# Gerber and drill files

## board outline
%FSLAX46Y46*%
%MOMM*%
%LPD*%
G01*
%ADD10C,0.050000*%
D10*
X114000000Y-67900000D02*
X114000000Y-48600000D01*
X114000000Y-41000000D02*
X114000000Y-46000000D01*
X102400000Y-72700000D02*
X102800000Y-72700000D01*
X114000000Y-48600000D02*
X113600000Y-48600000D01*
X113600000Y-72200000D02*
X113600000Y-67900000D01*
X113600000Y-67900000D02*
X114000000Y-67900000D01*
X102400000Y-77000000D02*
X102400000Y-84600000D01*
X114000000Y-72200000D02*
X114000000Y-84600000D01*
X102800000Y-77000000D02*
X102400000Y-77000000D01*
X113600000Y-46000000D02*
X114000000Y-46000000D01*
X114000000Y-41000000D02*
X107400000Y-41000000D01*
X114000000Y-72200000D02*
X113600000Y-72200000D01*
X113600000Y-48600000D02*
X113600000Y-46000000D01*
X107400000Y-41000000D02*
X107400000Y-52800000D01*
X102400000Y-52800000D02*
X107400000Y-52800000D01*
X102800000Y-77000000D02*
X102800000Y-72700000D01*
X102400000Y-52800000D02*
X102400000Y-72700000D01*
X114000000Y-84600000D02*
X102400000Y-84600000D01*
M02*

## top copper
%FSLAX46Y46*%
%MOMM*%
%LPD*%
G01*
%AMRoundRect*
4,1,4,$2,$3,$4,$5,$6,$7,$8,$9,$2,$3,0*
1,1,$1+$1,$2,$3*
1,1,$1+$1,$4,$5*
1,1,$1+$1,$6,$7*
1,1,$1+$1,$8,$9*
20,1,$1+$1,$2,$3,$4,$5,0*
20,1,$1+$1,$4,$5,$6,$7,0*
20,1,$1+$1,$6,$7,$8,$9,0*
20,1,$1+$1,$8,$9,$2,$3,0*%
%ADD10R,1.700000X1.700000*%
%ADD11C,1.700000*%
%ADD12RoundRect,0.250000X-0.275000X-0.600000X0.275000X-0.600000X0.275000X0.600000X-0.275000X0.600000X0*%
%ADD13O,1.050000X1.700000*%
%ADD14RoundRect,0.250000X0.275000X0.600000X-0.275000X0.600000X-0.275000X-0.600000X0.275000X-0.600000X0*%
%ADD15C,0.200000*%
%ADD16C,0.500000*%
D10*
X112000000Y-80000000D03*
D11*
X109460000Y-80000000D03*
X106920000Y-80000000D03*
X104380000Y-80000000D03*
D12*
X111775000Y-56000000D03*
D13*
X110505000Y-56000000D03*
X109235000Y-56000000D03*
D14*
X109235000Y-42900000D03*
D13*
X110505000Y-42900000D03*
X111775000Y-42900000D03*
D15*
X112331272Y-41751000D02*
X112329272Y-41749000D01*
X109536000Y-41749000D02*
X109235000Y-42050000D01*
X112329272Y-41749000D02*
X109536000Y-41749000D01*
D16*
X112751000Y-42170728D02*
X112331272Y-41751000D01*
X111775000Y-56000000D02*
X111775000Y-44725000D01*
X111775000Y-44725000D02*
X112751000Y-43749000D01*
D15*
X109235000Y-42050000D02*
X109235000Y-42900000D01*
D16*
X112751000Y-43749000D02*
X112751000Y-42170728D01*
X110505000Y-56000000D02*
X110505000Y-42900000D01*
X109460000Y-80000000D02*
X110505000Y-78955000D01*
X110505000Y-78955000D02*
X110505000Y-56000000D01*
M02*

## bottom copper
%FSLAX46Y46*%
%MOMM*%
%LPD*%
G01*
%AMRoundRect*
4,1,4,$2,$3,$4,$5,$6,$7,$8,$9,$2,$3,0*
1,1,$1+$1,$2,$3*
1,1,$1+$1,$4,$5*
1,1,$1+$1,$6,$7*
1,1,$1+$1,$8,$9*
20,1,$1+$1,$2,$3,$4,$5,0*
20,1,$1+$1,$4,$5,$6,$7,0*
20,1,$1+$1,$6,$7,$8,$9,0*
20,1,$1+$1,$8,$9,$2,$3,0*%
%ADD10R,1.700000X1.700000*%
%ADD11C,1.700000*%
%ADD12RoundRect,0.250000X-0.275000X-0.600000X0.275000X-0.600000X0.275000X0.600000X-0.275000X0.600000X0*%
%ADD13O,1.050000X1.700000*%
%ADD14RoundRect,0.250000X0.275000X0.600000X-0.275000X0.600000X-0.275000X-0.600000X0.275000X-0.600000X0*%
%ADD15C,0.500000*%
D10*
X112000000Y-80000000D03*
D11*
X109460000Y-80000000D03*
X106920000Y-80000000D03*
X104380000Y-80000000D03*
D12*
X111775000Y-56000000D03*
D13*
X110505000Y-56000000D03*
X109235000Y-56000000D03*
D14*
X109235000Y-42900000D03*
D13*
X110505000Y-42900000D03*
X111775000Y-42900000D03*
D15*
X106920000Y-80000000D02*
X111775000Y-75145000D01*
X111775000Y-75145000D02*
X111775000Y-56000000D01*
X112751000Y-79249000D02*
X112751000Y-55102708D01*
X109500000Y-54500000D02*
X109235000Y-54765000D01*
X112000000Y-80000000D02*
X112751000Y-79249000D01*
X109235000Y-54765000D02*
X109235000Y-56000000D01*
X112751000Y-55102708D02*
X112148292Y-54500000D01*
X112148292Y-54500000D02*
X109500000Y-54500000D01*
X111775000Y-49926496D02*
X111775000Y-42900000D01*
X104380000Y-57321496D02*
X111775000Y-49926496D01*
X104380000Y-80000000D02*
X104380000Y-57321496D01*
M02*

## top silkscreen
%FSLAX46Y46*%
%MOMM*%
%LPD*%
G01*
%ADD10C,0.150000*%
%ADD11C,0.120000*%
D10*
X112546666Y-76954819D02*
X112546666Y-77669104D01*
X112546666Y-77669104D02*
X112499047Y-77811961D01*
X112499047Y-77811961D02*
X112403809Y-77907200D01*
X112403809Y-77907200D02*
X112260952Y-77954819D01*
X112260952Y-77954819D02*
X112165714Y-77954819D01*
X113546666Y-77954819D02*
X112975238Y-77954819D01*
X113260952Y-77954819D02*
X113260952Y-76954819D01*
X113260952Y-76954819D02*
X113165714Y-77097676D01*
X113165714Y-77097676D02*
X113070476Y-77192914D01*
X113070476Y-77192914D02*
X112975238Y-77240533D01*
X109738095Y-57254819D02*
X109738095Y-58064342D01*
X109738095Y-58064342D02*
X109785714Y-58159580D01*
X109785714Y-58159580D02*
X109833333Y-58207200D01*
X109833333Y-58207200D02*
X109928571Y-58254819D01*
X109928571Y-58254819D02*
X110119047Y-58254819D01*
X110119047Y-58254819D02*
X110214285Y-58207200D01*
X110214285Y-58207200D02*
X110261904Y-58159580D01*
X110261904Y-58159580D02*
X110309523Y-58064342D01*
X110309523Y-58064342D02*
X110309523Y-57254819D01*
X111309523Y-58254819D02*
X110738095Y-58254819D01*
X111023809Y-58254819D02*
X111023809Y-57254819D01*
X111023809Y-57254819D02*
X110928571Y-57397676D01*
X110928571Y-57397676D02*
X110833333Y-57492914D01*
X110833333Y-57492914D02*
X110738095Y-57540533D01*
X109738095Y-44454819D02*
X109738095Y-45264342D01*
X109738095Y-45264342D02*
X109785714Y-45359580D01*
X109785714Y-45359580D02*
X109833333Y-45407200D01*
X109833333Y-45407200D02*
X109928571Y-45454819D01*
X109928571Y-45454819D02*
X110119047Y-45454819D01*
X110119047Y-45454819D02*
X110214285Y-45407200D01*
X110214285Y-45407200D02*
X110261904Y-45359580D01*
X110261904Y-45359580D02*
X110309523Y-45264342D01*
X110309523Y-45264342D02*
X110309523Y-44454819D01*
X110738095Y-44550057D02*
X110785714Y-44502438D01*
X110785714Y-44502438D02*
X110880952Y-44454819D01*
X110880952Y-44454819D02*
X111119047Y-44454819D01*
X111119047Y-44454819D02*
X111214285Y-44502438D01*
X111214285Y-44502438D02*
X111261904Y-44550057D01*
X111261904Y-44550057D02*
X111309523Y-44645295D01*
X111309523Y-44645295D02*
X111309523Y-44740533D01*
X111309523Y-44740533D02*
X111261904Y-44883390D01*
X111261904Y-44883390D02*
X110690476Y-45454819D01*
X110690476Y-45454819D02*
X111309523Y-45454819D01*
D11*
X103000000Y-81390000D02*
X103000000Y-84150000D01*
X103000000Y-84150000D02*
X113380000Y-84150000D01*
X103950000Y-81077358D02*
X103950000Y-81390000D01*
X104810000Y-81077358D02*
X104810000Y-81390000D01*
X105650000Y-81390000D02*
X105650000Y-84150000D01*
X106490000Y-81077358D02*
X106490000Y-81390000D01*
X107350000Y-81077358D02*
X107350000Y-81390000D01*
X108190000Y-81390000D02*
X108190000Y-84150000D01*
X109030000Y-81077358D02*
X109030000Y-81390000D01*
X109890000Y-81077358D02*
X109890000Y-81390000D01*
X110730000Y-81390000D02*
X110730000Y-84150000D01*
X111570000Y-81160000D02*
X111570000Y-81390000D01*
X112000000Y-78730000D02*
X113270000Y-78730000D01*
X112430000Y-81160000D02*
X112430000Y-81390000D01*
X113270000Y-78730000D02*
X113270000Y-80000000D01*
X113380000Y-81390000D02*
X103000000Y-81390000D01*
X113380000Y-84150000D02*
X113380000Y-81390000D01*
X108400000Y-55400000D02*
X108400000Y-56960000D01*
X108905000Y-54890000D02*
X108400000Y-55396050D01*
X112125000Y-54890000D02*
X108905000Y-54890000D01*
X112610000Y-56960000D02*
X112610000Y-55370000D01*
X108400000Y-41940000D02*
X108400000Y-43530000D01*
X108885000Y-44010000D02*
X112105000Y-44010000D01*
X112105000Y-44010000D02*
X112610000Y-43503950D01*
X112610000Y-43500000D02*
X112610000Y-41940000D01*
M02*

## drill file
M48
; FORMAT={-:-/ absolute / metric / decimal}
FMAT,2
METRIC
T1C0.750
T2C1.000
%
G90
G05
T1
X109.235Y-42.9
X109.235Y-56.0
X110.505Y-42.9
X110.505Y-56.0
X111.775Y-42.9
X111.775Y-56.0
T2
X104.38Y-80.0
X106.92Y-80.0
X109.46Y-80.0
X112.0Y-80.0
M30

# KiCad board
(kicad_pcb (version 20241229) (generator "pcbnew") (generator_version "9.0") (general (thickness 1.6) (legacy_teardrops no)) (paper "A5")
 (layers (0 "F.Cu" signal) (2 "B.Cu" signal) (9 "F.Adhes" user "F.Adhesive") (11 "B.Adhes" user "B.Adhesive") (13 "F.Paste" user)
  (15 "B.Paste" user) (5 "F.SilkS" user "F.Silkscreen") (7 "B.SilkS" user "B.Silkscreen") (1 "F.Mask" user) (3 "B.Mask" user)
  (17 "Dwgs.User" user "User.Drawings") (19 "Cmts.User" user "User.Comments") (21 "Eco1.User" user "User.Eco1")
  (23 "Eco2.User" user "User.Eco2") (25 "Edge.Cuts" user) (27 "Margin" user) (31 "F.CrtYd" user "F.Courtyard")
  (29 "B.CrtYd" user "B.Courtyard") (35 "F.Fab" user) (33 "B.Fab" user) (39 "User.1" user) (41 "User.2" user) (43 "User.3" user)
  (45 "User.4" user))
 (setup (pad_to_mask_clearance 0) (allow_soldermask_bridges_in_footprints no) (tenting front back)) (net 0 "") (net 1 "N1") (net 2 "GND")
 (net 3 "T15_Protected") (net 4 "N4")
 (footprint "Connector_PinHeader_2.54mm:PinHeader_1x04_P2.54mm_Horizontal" (layer "F.Cu") (at 112 80 -90)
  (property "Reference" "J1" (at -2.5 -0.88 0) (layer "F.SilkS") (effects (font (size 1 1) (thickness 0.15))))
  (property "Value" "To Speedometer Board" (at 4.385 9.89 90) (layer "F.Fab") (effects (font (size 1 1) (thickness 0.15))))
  (fp_line (start 1.39 9) (end 4.15 9) (stroke (width 0.12) (type solid)) (layer "F.SilkS"))
  (fp_line (start 4.15 9) (end 4.15 -1.38) (stroke (width 0.12) (type solid)) (layer "F.SilkS"))
  (fp_line (start 1.077358 8.05) (end 1.39 8.05) (stroke (width 0.12) (type solid)) (layer "F.SilkS"))
  (fp_line (start 1.077358 7.19) (end 1.39 7.19) (stroke (width 0.12) (type solid)) (layer "F.SilkS"))
  (fp_line (start 1.39 6.35) (end 4.15 6.35) (stroke (width 0.12) (type solid)) (layer "F.SilkS"))
  (fp_line (start 1.077358 5.51) (end 1.39 5.51) (stroke (width 0.12) (type solid)) (layer "F.SilkS"))
  (fp_line (start 1.077358 4.65) (end 1.39 4.65) (stroke (width 0.12) (type solid)) (layer "F.SilkS"))
  (fp_line (start 1.39 3.81) (end 4.15 3.81) (stroke (width 0.12) (type solid)) (layer "F.SilkS"))
  (fp_line (start 1.077358 2.97) (end 1.39 2.97) (stroke (width 0.12) (type solid)) (layer "F.SilkS"))
  (fp_line (start 1.077358 2.11) (end 1.39 2.11) (stroke (width 0.12) (type solid)) (layer "F.SilkS"))
  (fp_line (start 1.39 1.27) (end 4.15 1.27) (stroke (width 0.12) (type solid)) (layer "F.SilkS"))
  (fp_line (start 1.16 0.43) (end 1.39 0.43) (stroke (width 0.12) (type solid)) (layer "F.SilkS"))
  (fp_line (start -1.27 0) (end -1.27 -1.27) (stroke (width 0.12) (type solid)) (layer "F.SilkS"))
  (fp_line (start 1.16 -0.43) (end 1.39 -0.43) (stroke (width 0.12) (type solid)) (layer "F.SilkS"))
  (fp_line (start -1.27 -1.27) (end 0 -1.27) (stroke (width 0.12) (type solid)) (layer "F.SilkS"))
  (fp_line (start 1.39 -1.38) (end 1.39 9) (stroke (width 0.12) (type solid)) (layer "F.SilkS"))
  (fp_line (start 4.15 -1.38) (end 1.39 -1.38) (stroke (width 0.12) (type solid)) (layer "F.SilkS"))
  (pad "1" thru_hole rect (at 0 0 270) (size 1.7 1.7) (drill 1) (layers "*.Cu" "*.Mask") (remove_unused_layers no) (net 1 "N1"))
  (pad "2" thru_hole circle (at 0 2.54 270) (size 1.7 1.7) (drill 1) (layers "*.Cu" "*.Mask") (remove_unused_layers no) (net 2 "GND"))
  (pad "3" thru_hole circle (at 0 5.08 270) (size 1.7 1.7) (drill 1) (layers "*.Cu" "*.Mask") (remove_unused_layers no)
   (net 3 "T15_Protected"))
  (pad "4" thru_hole circle (at 0 7.62 270) (size 1.7 1.7) (drill 1) (layers "*.Cu" "*.Mask") (remove_unused_layers no) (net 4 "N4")))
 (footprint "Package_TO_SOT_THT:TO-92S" (layer "F.Cu") (at 111.775 56 180)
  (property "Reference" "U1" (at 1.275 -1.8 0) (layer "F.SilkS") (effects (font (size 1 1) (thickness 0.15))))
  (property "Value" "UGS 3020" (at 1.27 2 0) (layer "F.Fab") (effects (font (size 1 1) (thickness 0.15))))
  (fp_line (start 3.375 0.6) (end 3.375 -0.96) (stroke (width 0.12) (type solid)) (layer "F.SilkS"))
  (fp_line (start 2.87 1.11) (end 3.375 0.60395) (stroke (width 0.12) (type solid)) (layer "F.SilkS"))
  (fp_line (start -0.35 1.11) (end 2.87 1.11) (stroke (width 0.12) (type solid)) (layer "F.SilkS"))
  (fp_line (start -0.835 -0.96) (end -0.835 0.63) (stroke (width 0.12) (type solid)) (layer "F.SilkS"))
  (pad "1" thru_hole roundrect (at 0 0) (size 1.05 1.7) (drill 0.75) (layers "*.Cu" "*.Mask") (remove_unused_layers no)
   (roundrect_rratio 0.2380952381) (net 3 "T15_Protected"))
  (pad "2" thru_hole oval (at 1.27 0) (size 1.05 1.7) (drill 0.75) (layers "*.Cu" "*.Mask") (remove_unused_layers no) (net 2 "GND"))
  (pad "3" thru_hole oval (at 2.54 0) (size 1.05 1.7) (drill 0.75) (layers "*.Cu" "*.Mask") (remove_unused_layers no) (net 1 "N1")))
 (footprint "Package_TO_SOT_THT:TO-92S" (layer "F.Cu") (at 109.235 42.9)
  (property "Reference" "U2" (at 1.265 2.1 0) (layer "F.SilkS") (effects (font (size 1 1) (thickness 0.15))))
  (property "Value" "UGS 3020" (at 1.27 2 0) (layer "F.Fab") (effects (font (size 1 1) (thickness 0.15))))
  (fp_line (start -0.835 -0.96) (end -0.835 0.63) (stroke (width 0.12) (type solid)) (layer "F.SilkS"))
  (fp_line (start -0.35 1.11) (end 2.87 1.11) (stroke (width 0.12) (type solid)) (layer "F.SilkS"))
  (fp_line (start 2.87 1.11) (end 3.375 0.60395) (stroke (width 0.12) (type solid)) (layer "F.SilkS"))
  (fp_line (start 3.375 0.6) (end 3.375 -0.96) (stroke (width 0.12) (type solid)) (layer "F.SilkS"))
  (pad "1" thru_hole roundrect (at 0 0 180) (size 1.05 1.7) (drill 0.75) (layers "*.Cu" "*.Mask") (remove_unused_layers no)
   (roundrect_rratio 0.2380952381) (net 3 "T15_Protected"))
  (pad "2" thru_hole oval (at 1.27 0 180) (size 1.05 1.7) (drill 0.75) (layers "*.Cu" "*.Mask") (remove_unused_layers no) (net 2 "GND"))
  (pad "3" thru_hole oval (at 2.54 0 180) (size 1.05 1.7) (drill 0.75) (layers "*.Cu" "*.Mask") (remove_unused_layers no) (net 4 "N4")))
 (gr_line (start 114 67.9) (end 114 48.6) (stroke (width 0.05) (type solid)) (layer "Edge.Cuts"))
 (gr_line (start 114 41) (end 114 46) (stroke (width 0.05) (type default)) (layer "Edge.Cuts"))
 (gr_line (start 102.4 72.7) (end 102.8 72.7) (stroke (width 0.05) (type solid)) (layer "Edge.Cuts"))
 (gr_line (start 114 48.6) (end 113.6 48.6) (stroke (width 0.05) (type solid)) (layer "Edge.Cuts"))
 (gr_line (start 113.6 72.2) (end 113.6 67.9) (stroke (width 0.05) (type solid)) (layer "Edge.Cuts"))
 (gr_line (start 113.6 67.9) (end 114 67.9) (stroke (width 0.05) (type solid)) (layer "Edge.Cuts"))
 (gr_line (start 102.4 77) (end 102.4 84.6) (stroke (width 0.05) (type solid)) (layer "Edge.Cuts"))
 (gr_line (start 114 72.2) (end 114 84.6) (stroke (width 0.05) (type solid)) (layer "Edge.Cuts"))
 (gr_line (start 102.8 77) (end 102.4 77) (stroke (width 0.05) (type solid)) (layer "Edge.Cuts"))
 (gr_line (start 113.6 46) (end 114 46) (stroke (width 0.05) (type solid)) (layer "Edge.Cuts"))
 (gr_line (start 114 41) (end 107.4 41) (stroke (width 0.05) (type solid)) (layer "Edge.Cuts"))
 (gr_line (start 114 72.2) (end 113.6 72.2) (stroke (width 0.05) (type solid)) (layer "Edge.Cuts"))
 (gr_line (start 113.6 48.6) (end 113.6 46) (stroke (width 0.05) (type solid)) (layer "Edge.Cuts"))
 (gr_line (start 107.4 41) (end 107.4 52.8) (stroke (width 0.05) (type solid)) (layer "Edge.Cuts"))
 (gr_line (start 102.4 52.8) (end 107.4 52.8) (stroke (width 0.05) (type solid)) (layer "Edge.Cuts"))
 (gr_line (start 102.8 77) (end 102.8 72.7) (stroke (width 0.05) (type solid)) (layer "Edge.Cuts"))
 (gr_line (start 102.4 52.8) (end 102.4 72.7) (stroke (width 0.05) (type solid)) (layer "Edge.Cuts"))
 (gr_line (start 114 84.6) (end 102.4 84.6) (stroke (width 0.05) (type default)) (layer "Edge.Cuts"))
 (segment (start 112.331272 41.751) (end 112.329272 41.749) (width 0.2) (layer "F.Cu") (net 3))
 (segment (start 109.536 41.749) (end 109.235 42.05) (width 0.2) (layer "F.Cu") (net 3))
 (segment (start 112.329272 41.749) (end 109.536 41.749) (width 0.2) (layer "F.Cu") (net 3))
 (segment (start 112.751 42.170728) (end 112.331272 41.751) (width 0.5) (layer "F.Cu") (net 3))
 (segment (start 111.775 56) (end 111.775 44.725) (width 0.5) (layer "F.Cu") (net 3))
 (segment (start 111.775 44.725) (end 112.751 43.749) (width 0.5) (layer "F.Cu") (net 3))
 (segment (start 109.235 42.05) (end 109.235 42.9) (width 0.2) (layer "F.Cu") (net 3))
 (segment (start 112.751 43.749) (end 112.751 42.170728) (width 0.5) (layer "F.Cu") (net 3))
 (segment (start 106.92 80) (end 111.775 75.145) (width 0.5) (layer "B.Cu") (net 3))
 (segment (start 111.775 75.145) (end 111.775 56) (width 0.5) (layer "B.Cu") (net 3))
 (segment (start 110.505 56) (end 110.505 42.9) (width 0.5) (layer "F.Cu") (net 2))
 (segment (start 109.46 80) (end 110.505 78.955) (width 0.5) (layer "F.Cu") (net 2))
 (segment (start 110.505 78.955) (end 110.505 56) (width 0.5) (layer "F.Cu") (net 2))
 (segment (start 112.751 79.249) (end 112.751 55.102708) (width 0.5) (layer "B.Cu") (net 1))
 (segment (start 109.5 54.5) (end 109.235 54.765) (width 0.5) (layer "B.Cu") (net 1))
 (segment (start 112 80) (end 112.751 79.249) (width 0.5) (layer "B.Cu") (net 1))
 (segment (start 109.235 54.765) (end 109.235 56) (width 0.5) (layer "B.Cu") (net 1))
 (segment (start 112.751 55.102708) (end 112.148292 54.5) (width 0.5) (layer "B.Cu") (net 1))
 (segment (start 112.148292 54.5) (end 109.5 54.5) (width 0.5) (layer "B.Cu") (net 1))
 (segment (start 111.775 49.926496) (end 111.775 42.9) (width 0.5) (layer "B.Cu") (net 4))
 (segment (start 104.38 57.321496) (end 111.775 49.926496) (width 0.5) (layer "B.Cu") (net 4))
 (segment (start 104.38 80) (end 104.38 57.321496) (width 0.5) (layer "B.Cu") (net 4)))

